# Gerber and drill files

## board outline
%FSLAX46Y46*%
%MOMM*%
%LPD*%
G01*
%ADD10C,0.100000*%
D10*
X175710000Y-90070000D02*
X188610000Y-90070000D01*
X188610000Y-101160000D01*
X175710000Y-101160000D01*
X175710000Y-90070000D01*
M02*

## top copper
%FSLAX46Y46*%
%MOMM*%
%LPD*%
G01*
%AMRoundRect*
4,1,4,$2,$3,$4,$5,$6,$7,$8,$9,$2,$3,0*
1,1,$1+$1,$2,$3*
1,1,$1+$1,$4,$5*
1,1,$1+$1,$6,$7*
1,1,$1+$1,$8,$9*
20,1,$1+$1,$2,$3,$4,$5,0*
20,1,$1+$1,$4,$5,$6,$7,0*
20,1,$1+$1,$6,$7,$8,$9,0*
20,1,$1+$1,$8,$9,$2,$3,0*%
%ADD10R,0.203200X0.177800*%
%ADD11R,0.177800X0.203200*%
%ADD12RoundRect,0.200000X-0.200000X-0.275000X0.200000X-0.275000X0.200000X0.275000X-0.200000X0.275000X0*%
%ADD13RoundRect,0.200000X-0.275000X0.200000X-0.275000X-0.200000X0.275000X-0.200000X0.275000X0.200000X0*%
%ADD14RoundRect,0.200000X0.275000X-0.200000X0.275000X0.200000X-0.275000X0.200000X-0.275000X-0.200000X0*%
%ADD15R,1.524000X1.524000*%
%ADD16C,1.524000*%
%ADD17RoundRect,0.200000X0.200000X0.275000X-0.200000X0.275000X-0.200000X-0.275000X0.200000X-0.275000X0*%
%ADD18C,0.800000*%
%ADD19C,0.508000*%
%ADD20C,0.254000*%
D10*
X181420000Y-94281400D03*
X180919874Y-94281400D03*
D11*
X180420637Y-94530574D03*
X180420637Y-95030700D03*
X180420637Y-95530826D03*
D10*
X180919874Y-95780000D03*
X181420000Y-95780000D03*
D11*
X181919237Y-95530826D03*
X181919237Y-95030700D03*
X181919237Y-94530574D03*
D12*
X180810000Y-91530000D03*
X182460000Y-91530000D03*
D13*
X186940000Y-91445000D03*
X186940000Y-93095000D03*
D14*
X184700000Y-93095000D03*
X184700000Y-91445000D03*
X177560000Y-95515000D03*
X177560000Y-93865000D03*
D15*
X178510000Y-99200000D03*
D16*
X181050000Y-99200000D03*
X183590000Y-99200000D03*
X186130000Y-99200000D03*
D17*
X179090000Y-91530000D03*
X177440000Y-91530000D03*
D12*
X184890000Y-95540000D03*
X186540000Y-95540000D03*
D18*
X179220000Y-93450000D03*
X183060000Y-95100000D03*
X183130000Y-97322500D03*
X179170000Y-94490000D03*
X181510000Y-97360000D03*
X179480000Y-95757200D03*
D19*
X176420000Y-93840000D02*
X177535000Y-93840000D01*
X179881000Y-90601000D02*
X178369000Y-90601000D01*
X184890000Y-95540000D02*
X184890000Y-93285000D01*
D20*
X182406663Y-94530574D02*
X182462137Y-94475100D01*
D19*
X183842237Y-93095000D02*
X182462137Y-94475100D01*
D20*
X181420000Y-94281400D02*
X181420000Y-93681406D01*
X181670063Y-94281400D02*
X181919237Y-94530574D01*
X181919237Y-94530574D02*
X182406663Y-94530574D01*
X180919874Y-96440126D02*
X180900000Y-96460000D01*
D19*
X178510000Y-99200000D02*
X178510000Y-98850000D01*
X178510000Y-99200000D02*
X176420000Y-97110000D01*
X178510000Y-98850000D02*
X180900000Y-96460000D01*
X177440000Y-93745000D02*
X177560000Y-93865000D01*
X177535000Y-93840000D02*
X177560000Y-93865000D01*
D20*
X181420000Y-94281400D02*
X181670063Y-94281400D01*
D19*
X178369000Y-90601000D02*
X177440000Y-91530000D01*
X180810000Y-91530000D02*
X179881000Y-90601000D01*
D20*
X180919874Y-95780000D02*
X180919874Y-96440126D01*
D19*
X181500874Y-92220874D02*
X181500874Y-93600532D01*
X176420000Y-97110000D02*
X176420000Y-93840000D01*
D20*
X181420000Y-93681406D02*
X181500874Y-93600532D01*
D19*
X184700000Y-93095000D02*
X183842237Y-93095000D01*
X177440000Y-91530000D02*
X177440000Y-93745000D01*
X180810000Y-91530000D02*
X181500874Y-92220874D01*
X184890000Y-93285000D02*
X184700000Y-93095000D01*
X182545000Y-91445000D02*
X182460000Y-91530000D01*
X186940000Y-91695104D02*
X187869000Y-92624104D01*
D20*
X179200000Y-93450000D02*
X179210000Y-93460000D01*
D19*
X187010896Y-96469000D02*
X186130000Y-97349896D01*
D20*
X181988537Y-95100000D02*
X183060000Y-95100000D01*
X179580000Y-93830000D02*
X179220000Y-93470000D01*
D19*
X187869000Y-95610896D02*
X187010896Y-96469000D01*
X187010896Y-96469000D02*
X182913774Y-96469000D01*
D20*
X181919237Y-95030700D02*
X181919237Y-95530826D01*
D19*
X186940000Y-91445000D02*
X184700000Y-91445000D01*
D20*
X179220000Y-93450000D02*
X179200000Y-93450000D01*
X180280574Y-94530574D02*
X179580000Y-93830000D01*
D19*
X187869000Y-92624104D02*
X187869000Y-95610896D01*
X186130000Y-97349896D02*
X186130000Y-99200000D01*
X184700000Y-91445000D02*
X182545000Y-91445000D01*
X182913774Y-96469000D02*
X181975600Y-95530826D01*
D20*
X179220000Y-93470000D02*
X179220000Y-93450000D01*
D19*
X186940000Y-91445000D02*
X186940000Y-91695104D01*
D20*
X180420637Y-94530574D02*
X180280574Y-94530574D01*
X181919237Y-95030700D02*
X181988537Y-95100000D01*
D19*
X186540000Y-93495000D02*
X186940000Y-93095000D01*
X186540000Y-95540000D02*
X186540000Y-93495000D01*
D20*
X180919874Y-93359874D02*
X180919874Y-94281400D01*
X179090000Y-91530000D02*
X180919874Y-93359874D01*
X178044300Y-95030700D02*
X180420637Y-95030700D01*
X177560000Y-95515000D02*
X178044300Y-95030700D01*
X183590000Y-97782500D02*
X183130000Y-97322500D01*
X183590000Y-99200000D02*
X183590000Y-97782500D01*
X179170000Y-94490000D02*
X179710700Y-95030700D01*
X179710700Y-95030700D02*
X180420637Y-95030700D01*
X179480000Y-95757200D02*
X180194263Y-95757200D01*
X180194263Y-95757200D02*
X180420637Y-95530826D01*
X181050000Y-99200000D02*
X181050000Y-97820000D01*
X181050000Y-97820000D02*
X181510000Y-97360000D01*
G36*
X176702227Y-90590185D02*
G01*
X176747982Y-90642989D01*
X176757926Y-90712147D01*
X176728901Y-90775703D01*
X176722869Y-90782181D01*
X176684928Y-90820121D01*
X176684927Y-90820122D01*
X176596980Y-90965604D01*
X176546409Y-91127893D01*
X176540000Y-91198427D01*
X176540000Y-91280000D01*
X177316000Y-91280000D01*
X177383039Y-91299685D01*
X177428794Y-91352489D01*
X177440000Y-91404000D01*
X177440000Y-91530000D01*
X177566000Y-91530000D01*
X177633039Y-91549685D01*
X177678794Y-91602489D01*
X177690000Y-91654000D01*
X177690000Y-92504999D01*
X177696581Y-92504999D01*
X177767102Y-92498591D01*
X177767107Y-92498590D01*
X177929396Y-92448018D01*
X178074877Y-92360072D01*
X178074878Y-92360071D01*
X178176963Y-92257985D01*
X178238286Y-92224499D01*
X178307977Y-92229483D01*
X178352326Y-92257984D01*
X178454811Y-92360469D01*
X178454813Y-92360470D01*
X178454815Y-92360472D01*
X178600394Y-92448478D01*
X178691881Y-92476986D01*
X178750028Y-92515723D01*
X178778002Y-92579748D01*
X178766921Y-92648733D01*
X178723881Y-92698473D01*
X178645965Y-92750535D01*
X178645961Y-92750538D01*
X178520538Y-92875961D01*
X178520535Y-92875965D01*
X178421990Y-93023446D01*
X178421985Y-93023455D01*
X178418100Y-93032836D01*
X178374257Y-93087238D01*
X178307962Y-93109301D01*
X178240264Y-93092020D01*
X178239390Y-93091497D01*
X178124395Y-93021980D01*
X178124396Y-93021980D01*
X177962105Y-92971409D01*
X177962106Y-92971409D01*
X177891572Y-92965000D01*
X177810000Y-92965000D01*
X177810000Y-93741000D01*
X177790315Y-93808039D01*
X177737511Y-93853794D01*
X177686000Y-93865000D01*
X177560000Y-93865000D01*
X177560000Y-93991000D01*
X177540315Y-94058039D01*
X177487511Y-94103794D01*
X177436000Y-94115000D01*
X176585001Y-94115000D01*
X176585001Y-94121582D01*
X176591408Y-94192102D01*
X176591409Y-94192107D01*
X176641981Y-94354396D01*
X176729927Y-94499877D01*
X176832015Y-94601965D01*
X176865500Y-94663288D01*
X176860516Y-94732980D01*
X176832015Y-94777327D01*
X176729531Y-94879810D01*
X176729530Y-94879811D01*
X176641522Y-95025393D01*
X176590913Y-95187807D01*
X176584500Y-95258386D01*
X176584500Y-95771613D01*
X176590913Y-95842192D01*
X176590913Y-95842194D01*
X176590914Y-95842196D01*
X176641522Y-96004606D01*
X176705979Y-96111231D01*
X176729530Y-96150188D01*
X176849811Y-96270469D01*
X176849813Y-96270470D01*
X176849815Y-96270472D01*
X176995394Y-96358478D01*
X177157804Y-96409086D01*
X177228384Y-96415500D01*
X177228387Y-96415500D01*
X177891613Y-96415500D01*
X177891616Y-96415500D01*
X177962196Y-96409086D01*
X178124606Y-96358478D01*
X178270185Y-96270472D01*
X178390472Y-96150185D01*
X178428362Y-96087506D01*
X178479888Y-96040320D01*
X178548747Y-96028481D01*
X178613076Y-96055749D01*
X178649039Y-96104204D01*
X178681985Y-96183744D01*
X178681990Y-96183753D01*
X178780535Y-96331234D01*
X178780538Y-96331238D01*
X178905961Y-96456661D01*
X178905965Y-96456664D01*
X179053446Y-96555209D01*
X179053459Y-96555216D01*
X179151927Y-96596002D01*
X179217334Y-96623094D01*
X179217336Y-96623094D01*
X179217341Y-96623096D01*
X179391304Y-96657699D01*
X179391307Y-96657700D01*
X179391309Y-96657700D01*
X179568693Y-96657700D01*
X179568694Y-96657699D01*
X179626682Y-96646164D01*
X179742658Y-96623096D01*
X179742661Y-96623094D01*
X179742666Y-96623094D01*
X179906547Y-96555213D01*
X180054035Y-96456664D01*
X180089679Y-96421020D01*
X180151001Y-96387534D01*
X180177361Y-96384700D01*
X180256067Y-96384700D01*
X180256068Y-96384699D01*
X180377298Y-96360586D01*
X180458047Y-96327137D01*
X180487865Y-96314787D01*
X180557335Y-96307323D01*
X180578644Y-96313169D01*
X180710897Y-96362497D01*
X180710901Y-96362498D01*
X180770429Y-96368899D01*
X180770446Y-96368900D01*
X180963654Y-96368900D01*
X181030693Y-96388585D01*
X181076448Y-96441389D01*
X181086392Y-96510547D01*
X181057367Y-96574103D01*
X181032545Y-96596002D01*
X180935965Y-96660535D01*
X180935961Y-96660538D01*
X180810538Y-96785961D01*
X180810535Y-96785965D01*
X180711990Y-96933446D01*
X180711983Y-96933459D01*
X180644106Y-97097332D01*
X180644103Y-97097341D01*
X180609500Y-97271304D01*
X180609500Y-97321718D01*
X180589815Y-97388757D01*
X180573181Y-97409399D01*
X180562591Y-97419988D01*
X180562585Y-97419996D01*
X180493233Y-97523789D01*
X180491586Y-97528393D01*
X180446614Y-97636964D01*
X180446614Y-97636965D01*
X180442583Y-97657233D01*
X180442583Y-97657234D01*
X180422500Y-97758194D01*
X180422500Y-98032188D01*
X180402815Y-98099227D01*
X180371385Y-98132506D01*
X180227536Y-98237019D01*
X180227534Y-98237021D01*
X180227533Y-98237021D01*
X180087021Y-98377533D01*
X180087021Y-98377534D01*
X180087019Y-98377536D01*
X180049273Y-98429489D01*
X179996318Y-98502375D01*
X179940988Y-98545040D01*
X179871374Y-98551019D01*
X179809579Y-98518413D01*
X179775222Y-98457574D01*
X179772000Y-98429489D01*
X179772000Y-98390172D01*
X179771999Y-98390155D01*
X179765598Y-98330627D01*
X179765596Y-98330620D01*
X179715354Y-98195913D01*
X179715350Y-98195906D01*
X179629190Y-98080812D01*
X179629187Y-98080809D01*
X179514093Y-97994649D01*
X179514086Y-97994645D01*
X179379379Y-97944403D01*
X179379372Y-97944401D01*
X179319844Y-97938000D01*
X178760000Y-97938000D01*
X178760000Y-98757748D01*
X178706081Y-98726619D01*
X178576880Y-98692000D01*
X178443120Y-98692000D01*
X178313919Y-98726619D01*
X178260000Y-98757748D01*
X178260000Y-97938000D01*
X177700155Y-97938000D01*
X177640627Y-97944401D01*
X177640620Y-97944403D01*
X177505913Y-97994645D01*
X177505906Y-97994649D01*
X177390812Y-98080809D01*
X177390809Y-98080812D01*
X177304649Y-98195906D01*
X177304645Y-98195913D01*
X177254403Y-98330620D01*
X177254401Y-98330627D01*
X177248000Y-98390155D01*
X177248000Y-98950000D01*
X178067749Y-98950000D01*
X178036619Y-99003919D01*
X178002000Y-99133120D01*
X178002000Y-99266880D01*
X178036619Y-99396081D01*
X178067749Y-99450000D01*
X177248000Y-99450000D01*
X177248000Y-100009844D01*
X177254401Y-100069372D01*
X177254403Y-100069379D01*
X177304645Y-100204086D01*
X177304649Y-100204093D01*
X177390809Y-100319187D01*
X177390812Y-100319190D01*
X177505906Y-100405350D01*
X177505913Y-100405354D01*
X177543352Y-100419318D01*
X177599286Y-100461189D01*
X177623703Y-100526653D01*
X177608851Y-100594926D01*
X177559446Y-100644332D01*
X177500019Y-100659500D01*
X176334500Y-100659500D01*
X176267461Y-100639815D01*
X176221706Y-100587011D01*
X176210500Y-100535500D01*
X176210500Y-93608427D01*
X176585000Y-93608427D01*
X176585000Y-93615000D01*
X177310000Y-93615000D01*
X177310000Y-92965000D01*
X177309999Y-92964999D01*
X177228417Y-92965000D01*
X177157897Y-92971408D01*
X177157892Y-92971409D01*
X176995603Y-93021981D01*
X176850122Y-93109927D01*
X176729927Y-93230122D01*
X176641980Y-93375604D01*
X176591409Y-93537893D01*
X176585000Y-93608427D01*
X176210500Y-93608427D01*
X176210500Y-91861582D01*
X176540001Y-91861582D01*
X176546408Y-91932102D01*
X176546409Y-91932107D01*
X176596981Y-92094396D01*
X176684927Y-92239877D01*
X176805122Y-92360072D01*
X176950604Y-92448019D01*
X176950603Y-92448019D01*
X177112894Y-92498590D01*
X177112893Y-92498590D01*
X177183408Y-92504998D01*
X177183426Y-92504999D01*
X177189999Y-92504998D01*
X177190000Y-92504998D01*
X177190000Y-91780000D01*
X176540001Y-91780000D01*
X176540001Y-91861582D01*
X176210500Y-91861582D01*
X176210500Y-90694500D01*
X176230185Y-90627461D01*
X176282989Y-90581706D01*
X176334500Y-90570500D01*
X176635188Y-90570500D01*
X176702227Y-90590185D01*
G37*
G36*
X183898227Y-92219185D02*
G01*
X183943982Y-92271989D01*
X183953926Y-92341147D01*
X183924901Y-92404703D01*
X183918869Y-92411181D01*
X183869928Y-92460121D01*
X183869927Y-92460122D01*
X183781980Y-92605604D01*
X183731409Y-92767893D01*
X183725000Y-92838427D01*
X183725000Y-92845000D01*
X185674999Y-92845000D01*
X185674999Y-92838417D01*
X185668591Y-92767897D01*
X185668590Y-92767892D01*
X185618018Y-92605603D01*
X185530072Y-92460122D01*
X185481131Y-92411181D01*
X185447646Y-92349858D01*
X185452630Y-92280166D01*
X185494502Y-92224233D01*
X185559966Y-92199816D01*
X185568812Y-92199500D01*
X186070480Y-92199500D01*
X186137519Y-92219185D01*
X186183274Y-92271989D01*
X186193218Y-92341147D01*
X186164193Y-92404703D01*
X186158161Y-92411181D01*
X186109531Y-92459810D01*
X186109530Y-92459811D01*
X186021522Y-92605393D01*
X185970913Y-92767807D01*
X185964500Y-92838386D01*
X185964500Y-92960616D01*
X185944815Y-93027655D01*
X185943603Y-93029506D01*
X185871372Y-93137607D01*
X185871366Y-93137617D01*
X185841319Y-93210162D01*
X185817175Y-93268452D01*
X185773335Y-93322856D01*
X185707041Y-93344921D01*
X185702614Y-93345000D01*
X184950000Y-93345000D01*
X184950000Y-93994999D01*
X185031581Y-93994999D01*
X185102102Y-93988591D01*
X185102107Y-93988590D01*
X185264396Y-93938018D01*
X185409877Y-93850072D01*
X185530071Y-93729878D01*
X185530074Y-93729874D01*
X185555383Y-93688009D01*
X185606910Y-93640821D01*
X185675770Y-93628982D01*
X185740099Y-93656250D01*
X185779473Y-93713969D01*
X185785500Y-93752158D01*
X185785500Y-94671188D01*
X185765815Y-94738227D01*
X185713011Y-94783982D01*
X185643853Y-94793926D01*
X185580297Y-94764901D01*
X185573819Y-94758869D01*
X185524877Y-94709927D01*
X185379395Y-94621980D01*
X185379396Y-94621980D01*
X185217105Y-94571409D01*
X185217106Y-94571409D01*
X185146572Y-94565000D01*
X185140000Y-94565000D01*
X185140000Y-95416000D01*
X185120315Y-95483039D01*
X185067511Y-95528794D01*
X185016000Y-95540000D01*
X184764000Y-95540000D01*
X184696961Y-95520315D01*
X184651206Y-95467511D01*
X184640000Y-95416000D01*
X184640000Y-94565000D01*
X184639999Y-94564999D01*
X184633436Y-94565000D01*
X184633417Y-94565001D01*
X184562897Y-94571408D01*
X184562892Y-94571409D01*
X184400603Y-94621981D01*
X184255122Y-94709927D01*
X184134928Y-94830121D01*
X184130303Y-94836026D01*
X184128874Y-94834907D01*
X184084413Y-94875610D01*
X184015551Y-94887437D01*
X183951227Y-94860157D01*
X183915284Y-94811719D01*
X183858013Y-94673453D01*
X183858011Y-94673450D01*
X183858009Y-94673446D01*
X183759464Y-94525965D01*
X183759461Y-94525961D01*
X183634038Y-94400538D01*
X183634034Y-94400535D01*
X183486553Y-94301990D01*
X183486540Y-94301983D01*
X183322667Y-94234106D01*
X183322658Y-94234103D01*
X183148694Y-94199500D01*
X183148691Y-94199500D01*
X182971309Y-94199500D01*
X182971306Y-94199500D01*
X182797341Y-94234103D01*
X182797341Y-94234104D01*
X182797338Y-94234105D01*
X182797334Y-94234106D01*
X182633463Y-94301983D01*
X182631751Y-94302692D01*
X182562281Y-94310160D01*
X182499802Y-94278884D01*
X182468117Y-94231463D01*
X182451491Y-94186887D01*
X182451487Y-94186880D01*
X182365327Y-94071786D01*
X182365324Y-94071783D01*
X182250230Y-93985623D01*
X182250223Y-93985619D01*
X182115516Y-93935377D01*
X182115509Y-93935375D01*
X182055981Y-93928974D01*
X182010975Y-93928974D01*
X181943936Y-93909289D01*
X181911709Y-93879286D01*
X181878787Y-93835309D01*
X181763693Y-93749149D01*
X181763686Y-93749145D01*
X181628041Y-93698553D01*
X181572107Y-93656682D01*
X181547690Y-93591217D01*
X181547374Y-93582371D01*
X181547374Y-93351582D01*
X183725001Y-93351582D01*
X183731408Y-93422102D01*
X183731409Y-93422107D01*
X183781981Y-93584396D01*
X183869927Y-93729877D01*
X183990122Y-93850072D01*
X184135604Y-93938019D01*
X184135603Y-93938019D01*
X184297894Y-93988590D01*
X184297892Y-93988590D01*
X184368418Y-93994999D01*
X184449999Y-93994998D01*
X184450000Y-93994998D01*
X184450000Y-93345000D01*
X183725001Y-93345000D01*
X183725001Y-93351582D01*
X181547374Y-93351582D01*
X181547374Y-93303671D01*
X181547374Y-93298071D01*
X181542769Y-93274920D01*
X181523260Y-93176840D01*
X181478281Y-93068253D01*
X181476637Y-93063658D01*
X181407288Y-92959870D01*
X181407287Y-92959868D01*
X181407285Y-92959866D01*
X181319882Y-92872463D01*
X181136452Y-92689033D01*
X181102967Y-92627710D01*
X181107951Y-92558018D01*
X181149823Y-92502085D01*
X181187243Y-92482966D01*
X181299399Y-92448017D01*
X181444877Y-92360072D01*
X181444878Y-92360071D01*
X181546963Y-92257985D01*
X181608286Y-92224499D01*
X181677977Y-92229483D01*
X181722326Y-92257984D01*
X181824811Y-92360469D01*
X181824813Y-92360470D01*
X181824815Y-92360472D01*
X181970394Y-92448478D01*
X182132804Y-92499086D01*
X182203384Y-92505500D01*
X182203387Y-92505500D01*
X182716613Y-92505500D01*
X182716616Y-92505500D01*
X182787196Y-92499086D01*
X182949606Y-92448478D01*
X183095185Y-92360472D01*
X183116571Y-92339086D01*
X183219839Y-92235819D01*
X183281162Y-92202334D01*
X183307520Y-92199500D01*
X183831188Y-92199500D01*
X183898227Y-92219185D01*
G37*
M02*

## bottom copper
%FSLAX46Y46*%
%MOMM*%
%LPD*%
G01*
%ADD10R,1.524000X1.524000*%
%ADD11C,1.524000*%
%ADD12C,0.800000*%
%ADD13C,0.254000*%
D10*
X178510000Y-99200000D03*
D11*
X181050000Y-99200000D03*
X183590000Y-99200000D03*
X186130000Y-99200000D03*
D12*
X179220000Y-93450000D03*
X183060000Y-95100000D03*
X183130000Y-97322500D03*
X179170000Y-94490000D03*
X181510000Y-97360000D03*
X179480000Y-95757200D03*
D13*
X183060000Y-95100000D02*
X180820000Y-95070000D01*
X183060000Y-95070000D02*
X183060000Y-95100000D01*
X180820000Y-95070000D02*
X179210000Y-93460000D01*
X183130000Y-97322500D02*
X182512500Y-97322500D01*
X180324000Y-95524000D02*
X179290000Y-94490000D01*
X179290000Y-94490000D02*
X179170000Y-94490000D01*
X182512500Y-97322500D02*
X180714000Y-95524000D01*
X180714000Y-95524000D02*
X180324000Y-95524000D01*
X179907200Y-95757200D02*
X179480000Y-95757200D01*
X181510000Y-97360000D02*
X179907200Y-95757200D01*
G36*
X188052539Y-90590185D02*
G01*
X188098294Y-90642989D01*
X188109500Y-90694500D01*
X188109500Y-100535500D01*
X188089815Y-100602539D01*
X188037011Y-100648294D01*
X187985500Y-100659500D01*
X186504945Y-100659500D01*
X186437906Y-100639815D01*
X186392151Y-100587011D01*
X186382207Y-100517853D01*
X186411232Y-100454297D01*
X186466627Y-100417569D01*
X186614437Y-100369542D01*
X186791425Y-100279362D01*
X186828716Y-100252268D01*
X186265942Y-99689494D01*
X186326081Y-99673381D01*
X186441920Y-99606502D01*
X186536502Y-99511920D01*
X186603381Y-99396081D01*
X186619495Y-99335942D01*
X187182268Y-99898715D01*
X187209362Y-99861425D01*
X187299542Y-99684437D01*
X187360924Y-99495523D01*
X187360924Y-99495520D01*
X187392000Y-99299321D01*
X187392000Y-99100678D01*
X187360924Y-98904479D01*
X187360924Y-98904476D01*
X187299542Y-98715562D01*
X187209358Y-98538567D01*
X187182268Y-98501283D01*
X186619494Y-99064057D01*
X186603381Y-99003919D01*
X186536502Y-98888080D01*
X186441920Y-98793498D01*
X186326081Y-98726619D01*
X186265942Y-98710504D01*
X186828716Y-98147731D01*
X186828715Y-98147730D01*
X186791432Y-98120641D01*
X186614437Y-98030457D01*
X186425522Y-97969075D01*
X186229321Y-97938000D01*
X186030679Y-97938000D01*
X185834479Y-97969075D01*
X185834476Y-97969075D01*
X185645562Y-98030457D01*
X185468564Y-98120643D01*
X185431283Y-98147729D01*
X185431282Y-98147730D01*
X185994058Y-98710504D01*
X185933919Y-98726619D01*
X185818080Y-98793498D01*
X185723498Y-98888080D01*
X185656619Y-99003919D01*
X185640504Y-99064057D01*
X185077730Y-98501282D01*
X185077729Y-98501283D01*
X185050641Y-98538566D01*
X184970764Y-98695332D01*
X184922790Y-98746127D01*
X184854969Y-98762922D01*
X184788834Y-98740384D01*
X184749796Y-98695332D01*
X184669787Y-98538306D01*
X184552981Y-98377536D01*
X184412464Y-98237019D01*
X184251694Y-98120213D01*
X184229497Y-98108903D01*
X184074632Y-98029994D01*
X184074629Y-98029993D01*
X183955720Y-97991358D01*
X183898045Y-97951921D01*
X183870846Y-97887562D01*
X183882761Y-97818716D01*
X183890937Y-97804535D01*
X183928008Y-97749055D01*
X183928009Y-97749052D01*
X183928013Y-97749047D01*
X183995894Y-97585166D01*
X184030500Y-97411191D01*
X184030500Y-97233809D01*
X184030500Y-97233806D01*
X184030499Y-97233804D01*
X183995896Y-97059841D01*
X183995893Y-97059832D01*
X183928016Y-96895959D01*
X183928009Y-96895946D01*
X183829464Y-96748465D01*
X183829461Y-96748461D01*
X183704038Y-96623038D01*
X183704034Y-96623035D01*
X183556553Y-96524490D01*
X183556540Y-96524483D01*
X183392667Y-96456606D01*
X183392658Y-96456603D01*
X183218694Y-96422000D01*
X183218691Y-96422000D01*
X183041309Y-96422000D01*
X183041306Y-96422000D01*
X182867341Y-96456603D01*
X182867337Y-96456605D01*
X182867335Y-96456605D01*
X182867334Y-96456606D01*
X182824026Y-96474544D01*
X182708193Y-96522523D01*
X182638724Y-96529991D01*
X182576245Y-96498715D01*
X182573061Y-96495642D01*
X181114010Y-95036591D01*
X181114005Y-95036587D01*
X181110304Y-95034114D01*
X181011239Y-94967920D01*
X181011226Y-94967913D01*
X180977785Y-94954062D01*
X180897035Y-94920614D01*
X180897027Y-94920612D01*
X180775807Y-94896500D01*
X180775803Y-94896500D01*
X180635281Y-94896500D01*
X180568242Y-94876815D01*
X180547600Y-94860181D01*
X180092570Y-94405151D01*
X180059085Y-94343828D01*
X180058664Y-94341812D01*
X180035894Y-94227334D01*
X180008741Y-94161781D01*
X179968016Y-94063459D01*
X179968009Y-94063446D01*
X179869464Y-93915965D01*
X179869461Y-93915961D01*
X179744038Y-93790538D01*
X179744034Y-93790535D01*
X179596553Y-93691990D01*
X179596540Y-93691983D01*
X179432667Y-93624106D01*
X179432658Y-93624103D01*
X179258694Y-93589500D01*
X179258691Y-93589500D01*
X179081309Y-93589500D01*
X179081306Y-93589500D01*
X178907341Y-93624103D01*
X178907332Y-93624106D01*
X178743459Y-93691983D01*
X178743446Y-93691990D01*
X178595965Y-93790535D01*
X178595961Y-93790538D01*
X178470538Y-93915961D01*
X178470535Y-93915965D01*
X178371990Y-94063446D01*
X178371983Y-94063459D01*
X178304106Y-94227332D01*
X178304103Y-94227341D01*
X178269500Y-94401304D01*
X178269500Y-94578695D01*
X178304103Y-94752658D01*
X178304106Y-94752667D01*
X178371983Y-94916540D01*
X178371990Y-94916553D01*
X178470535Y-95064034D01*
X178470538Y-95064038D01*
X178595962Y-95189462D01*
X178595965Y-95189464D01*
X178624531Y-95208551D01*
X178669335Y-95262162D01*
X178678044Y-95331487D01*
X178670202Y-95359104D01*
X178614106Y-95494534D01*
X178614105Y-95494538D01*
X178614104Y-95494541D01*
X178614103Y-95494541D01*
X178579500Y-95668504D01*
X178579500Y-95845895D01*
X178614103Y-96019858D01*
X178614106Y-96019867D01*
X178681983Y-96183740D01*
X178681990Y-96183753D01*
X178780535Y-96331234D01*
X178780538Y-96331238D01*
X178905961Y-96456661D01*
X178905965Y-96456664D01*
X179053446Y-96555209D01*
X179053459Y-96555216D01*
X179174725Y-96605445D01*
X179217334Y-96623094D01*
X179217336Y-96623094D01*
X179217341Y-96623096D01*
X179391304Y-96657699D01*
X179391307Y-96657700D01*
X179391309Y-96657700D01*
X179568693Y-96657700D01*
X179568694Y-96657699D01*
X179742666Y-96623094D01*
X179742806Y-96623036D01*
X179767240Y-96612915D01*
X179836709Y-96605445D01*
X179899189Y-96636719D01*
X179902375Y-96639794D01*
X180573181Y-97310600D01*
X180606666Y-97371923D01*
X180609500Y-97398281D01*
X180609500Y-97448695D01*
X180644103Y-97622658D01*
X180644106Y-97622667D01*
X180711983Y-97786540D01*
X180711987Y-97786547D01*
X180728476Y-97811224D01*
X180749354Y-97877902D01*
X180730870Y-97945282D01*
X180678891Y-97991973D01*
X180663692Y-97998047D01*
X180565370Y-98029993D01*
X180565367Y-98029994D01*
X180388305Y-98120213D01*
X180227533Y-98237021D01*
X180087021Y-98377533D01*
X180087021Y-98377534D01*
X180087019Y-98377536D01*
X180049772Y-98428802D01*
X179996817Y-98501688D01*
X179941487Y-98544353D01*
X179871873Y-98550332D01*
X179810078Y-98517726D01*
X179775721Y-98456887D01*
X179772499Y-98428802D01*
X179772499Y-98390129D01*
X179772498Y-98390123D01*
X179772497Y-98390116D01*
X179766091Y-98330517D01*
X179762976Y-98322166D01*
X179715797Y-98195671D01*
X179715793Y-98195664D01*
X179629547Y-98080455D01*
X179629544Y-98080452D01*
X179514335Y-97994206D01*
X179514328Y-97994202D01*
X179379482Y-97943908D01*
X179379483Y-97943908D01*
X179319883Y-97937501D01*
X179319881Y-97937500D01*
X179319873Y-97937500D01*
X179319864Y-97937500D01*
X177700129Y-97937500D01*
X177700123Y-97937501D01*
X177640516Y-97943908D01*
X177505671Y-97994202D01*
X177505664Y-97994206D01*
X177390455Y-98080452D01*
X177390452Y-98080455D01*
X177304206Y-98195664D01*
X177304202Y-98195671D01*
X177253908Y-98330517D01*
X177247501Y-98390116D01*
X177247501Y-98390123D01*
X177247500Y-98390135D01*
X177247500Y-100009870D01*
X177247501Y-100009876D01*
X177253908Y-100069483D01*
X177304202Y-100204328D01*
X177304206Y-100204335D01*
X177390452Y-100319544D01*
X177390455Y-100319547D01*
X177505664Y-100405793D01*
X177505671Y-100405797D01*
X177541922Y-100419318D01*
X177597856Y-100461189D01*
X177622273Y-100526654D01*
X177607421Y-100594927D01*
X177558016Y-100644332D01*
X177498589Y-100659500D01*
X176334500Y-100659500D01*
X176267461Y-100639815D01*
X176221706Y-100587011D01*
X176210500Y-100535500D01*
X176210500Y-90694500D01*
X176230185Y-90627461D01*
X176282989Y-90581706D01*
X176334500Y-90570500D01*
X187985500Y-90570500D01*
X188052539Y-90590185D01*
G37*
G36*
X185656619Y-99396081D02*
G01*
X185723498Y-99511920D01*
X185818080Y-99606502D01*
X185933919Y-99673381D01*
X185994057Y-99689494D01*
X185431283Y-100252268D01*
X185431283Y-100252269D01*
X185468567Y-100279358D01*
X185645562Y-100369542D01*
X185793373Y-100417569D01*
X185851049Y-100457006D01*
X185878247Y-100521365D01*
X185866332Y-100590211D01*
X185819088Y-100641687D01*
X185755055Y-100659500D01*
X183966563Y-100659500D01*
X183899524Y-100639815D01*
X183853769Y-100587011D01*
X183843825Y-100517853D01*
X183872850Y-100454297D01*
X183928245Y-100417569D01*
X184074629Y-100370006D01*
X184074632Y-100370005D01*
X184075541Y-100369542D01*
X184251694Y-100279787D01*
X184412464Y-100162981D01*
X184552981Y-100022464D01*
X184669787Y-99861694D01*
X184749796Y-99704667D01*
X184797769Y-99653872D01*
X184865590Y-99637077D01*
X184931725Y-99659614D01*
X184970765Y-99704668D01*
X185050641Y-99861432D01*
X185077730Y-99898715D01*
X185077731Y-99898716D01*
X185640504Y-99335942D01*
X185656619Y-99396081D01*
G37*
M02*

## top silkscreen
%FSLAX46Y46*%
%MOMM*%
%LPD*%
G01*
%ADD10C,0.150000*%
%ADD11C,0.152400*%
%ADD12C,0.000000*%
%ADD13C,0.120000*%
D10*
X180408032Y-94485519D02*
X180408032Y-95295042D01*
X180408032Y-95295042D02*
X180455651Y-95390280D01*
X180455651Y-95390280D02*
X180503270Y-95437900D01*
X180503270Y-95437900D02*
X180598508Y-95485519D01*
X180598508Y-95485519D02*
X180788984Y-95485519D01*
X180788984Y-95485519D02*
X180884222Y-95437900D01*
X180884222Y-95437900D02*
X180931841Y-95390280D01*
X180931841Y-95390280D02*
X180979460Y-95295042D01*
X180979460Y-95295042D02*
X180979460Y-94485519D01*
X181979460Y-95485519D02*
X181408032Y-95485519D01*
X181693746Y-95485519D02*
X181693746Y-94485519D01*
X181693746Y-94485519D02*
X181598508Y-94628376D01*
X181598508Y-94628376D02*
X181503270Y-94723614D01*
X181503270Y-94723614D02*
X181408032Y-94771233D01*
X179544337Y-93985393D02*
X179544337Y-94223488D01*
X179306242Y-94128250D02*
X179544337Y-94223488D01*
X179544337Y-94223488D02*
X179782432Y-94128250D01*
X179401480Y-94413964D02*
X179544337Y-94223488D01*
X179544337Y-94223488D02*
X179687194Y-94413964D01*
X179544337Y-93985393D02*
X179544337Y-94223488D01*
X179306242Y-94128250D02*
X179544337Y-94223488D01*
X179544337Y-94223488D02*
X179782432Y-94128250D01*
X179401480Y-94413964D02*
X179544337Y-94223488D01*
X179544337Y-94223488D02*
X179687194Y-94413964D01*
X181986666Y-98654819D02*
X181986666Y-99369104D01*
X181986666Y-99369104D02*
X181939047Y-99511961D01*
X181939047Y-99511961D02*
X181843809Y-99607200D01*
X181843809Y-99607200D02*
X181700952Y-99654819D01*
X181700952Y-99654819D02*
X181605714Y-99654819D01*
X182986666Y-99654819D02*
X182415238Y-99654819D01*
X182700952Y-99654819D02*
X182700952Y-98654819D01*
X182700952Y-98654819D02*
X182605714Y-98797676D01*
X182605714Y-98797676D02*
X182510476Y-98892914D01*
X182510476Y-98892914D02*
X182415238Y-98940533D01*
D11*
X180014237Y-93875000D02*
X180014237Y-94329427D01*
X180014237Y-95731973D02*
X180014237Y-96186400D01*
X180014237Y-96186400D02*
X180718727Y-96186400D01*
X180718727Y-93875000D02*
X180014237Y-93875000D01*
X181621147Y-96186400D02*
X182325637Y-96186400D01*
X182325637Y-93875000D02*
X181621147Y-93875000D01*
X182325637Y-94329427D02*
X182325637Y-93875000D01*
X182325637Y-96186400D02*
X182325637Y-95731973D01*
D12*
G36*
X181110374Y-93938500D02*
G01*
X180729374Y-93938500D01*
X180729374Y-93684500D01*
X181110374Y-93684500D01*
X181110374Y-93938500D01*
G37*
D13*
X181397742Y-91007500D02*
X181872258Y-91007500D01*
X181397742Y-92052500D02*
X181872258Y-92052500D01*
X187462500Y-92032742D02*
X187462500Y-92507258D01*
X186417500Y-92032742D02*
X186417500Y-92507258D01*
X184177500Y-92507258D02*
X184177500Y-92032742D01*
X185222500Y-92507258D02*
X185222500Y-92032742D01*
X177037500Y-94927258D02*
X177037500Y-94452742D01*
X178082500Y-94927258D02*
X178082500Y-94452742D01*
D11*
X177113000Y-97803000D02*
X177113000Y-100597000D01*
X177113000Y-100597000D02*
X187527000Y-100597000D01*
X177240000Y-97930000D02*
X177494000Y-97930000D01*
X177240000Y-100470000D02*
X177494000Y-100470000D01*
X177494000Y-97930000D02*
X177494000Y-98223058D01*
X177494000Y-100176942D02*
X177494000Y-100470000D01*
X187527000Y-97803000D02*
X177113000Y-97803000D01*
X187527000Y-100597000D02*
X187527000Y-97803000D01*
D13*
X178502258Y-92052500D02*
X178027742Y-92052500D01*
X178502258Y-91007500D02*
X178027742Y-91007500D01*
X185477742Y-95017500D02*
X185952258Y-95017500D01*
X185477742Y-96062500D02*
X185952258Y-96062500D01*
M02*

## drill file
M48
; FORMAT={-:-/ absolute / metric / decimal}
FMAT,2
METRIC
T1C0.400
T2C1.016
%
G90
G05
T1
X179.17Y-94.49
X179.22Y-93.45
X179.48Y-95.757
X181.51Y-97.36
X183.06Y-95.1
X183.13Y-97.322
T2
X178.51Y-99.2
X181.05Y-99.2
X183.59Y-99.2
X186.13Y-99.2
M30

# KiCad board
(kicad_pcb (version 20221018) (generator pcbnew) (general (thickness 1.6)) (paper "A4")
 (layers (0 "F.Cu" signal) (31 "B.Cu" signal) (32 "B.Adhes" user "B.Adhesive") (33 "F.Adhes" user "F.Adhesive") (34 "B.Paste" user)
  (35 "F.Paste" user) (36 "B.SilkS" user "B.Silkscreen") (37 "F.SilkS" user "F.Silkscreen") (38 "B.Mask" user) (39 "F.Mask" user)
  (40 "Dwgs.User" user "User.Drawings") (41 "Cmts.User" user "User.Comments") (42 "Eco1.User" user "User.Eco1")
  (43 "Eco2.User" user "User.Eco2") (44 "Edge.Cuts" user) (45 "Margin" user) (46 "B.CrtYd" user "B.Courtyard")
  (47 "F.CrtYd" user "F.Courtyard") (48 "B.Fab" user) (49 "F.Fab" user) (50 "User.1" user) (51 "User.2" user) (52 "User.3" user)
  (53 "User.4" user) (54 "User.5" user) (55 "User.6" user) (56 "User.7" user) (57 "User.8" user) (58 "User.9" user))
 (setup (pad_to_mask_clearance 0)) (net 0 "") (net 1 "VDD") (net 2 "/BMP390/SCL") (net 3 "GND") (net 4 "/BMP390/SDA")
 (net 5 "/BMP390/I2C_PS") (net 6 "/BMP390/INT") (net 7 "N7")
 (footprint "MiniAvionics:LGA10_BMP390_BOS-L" (layer "F.Cu") (at 181.169937 95.0307)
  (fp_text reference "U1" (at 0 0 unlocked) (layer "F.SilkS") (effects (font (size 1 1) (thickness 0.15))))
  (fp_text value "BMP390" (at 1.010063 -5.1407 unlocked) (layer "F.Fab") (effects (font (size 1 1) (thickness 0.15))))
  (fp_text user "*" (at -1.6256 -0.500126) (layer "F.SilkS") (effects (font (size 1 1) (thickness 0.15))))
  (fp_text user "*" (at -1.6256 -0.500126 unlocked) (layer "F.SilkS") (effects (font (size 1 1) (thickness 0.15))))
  (fp_line (start -1.1557 -1.1557) (end -1.1557 -0.701273) (stroke (width 0.1524) (type solid)) (layer "F.SilkS"))
  (fp_line (start -1.1557 0.701273) (end -1.1557 1.1557) (stroke (width 0.1524) (type solid)) (layer "F.SilkS"))
  (fp_line (start -1.1557 1.1557) (end -0.45121 1.1557) (stroke (width 0.1524) (type solid)) (layer "F.SilkS"))
  (fp_line (start -0.45121 -1.1557) (end -1.1557 -1.1557) (stroke (width 0.1524) (type solid)) (layer "F.SilkS"))
  (fp_line (start 0.45121 1.1557) (end 1.1557 1.1557) (stroke (width 0.1524) (type solid)) (layer "F.SilkS"))
  (fp_line (start 1.1557 -1.1557) (end 0.45121 -1.1557) (stroke (width 0.1524) (type solid)) (layer "F.SilkS"))
  (fp_line (start 1.1557 -0.701273) (end 1.1557 -1.1557) (stroke (width 0.1524) (type solid)) (layer "F.SilkS"))
  (fp_line (start 1.1557 1.1557) (end 1.1557 0.701273) (stroke (width 0.1524) (type solid)) (layer "F.SilkS"))
  (fp_poly
   (pts (xy -0.440563 -1.0922) (xy -0.440563 -1.3462) (xy -0.059563 -1.3462) (xy -0.059563 -1.0922)) (stroke (width 0) (type solid))
   (fill solid) (layer "F.SilkS"))
  (pad "1" smd rect (at 0.250063 -0.7493) (size 0.2032 0.1778) (layers "F.Cu" "F.Paste" "F.Mask") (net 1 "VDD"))
  (pad "2" smd rect (at -0.250063 -0.7493) (size 0.2032 0.1778) (layers "F.Cu" "F.Paste" "F.Mask") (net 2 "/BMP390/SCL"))
  (pad "3" smd rect (at -0.7493 -0.500126 90) (size 0.2032 0.1778) (layers "F.Cu" "F.Paste" "F.Mask") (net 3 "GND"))
  (pad "4" smd rect (at -0.7493 0 90) (size 0.2032 0.1778) (layers "F.Cu" "F.Paste" "F.Mask") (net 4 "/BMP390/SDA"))
  (pad "5" smd rect (at -0.7493 0.500126 90) (size 0.2032 0.1778) (layers "F.Cu" "F.Paste" "F.Mask") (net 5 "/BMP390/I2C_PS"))
  (pad "6" smd rect (at -0.250063 0.7493) (size 0.2032 0.1778) (layers "F.Cu" "F.Paste" "F.Mask") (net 1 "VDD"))
  (pad "7" smd rect (at 0.250063 0.7493) (size 0.2032 0.1778) (layers "F.Cu" "F.Paste" "F.Mask") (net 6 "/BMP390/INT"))
  (pad "8" smd rect (at 0.7493 0.500126 90) (size 0.2032 0.1778) (layers "F.Cu" "F.Paste" "F.Mask") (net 3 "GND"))
  (pad "9" smd rect (at 0.7493 0 90) (size 0.2032 0.1778) (layers "F.Cu" "F.Paste" "F.Mask") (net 3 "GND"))
  (pad "10" smd rect (at 0.7493 -0.500126 90) (size 0.2032 0.1778) (layers "F.Cu" "F.Paste" "F.Mask") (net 1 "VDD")))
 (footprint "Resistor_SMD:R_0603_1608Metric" (layer "F.Cu") (at 181.635 91.53)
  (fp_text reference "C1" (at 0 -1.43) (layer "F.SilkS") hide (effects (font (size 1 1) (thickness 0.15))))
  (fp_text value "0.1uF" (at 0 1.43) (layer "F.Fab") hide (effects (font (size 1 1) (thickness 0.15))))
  (fp_line (start -0.237258 -0.5225) (end 0.237258 -0.5225) (stroke (width 0.12) (type solid)) (layer "F.SilkS"))
  (fp_line (start -0.237258 0.5225) (end 0.237258 0.5225) (stroke (width 0.12) (type solid)) (layer "F.SilkS"))
  (pad "1" smd roundrect (at -0.825 0) (size 0.8 0.95) (layers "F.Cu" "F.Paste" "F.Mask") (roundrect_rratio 0.25) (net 1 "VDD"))
  (pad "2" smd roundrect (at 0.825 0) (size 0.8 0.95) (layers "F.Cu" "F.Paste" "F.Mask") (roundrect_rratio 0.25) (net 3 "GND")))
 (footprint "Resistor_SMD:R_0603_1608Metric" (layer "F.Cu") (at 186.94 92.27 -90)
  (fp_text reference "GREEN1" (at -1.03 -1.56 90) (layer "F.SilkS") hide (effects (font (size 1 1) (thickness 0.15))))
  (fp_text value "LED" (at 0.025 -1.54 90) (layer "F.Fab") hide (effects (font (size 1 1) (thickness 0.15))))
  (fp_line (start -0.237258 -0.5225) (end 0.237258 -0.5225) (stroke (width 0.12) (type solid)) (layer "F.SilkS"))
  (fp_line (start -0.237258 0.5225) (end 0.237258 0.5225) (stroke (width 0.12) (type solid)) (layer "F.SilkS"))
  (pad "1" smd roundrect (at -0.825 0 270) (size 0.8 0.95) (layers "F.Cu" "F.Paste" "F.Mask") (roundrect_rratio 0.25) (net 3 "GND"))
  (pad "2" smd roundrect (at 0.825 0 270) (size 0.8 0.95) (layers "F.Cu" "F.Paste" "F.Mask") (roundrect_rratio 0.25) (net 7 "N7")))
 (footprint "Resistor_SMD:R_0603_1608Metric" (layer "F.Cu") (at 184.7 92.27 90)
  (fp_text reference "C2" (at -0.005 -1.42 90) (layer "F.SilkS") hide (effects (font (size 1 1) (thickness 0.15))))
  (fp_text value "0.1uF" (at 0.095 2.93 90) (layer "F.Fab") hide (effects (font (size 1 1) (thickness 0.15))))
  (fp_line (start -0.237258 -0.5225) (end 0.237258 -0.5225) (stroke (width 0.12) (type solid)) (layer "F.SilkS"))
  (fp_line (start -0.237258 0.5225) (end 0.237258 0.5225) (stroke (width 0.12) (type solid)) (layer "F.SilkS"))
  (pad "1" smd roundrect (at -0.825 0 90) (size 0.8 0.95) (layers "F.Cu" "F.Paste" "F.Mask") (roundrect_rratio 0.25) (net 1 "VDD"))
  (pad "2" smd roundrect (at 0.825 0 90) (size 0.8 0.95) (layers "F.Cu" "F.Paste" "F.Mask") (roundrect_rratio 0.25) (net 3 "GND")))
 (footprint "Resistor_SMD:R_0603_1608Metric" (layer "F.Cu") (at 177.56 94.69 90)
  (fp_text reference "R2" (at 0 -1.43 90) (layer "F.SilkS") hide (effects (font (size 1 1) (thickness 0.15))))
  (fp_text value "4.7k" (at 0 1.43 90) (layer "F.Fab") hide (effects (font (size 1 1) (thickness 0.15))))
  (fp_line (start -0.237258 -0.5225) (end 0.237258 -0.5225) (stroke (width 0.12) (type solid)) (layer "F.SilkS"))
  (fp_line (start -0.237258 0.5225) (end 0.237258 0.5225) (stroke (width 0.12) (type solid)) (layer "F.SilkS"))
  (pad "1" smd roundrect (at -0.825 0 90) (size 0.8 0.95) (layers "F.Cu" "F.Paste" "F.Mask") (roundrect_rratio 0.25) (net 4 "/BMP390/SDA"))
  (pad "2" smd roundrect (at 0.825 0 90) (size 0.8 0.95) (layers "F.Cu" "F.Paste" "F.Mask") (roundrect_rratio 0.25) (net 1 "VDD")))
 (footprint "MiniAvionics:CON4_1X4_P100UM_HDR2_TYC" (layer "F.Cu") (at 178.51 99.2)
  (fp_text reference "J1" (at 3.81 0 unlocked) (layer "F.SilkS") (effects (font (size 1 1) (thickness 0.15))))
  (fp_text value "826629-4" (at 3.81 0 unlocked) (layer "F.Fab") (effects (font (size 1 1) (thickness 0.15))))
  (fp_line (start -1.397 -1.397) (end -1.397 1.397) (stroke (width 0.1524) (type solid)) (layer "F.SilkS"))
  (fp_line (start -1.397 1.397) (end 9.017 1.397) (stroke (width 0.1524) (type solid)) (layer "F.SilkS"))
  (fp_line (start -1.27 -1.27) (end -1.016 -1.27) (stroke (width 0.1524) (type solid)) (layer "F.SilkS"))
  (fp_line (start -1.27 1.27) (end -1.016 1.27) (stroke (width 0.1524) (type solid)) (layer "F.SilkS"))
  (fp_line (start -1.016 -1.27) (end -1.016 -0.976942) (stroke (width 0.1524) (type solid)) (layer "F.SilkS"))
  (fp_line (start -1.016 0.976942) (end -1.016 1.27) (stroke (width 0.1524) (type solid)) (layer "F.SilkS"))
  (fp_line (start 9.017 -1.397) (end -1.397 -1.397) (stroke (width 0.1524) (type solid)) (layer "F.SilkS"))
  (fp_line (start 9.017 1.397) (end 9.017 -1.397) (stroke (width 0.1524) (type solid)) (layer "F.SilkS"))
  (pad "1" thru_hole rect (at 0 0) (size 1.524 1.524) (drill 1.016) (layers "*.Cu" "*.Mask") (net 1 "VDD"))
  (pad "2" thru_hole circle (at 2.54 0) (size 1.524 1.524) (drill 1.016) (layers "*.Cu" "*.Mask") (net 5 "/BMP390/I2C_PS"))
  (pad "3" thru_hole circle (at 5.08 0) (size 1.524 1.524) (drill 1.016) (layers "*.Cu" "*.Mask") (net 4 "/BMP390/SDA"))
  (pad "4" thru_hole circle (at 7.62 0) (size 1.524 1.524) (drill 1.016) (layers "*.Cu" "*.Mask") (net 3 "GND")))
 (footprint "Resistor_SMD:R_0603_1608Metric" (layer "F.Cu") (at 178.265 91.53 180)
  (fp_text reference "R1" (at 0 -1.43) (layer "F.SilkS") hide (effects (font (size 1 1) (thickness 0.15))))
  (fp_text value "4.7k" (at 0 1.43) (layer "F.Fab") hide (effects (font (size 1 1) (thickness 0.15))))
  (fp_line (start -0.237258 -0.5225) (end 0.237258 -0.5225) (stroke (width 0.12) (type solid)) (layer "F.SilkS"))
  (fp_line (start -0.237258 0.5225) (end 0.237258 0.5225) (stroke (width 0.12) (type solid)) (layer "F.SilkS"))
  (pad "1" smd roundrect (at -0.825 0 180) (size 0.8 0.95) (layers "F.Cu" "F.Paste" "F.Mask") (roundrect_rratio 0.25) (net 2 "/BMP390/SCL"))
  (pad "2" smd roundrect (at 0.825 0 180) (size 0.8 0.95) (layers "F.Cu" "F.Paste" "F.Mask") (roundrect_rratio 0.25) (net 1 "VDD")))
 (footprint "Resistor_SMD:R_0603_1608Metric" (layer "F.Cu") (at 185.715 95.54)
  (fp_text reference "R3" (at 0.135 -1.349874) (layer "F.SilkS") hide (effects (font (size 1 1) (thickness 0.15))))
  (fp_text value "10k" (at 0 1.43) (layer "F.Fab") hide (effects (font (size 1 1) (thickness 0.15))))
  (fp_line (start -0.237258 -0.5225) (end 0.237258 -0.5225) (stroke (width 0.12) (type solid)) (layer "F.SilkS"))
  (fp_line (start -0.237258 0.5225) (end 0.237258 0.5225) (stroke (width 0.12) (type solid)) (layer "F.SilkS"))
  (pad "1" smd roundrect (at -0.825 0) (size 0.8 0.95) (layers "F.Cu" "F.Paste" "F.Mask") (roundrect_rratio 0.25) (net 1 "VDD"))
  (pad "2" smd roundrect (at 0.825 0) (size 0.8 0.95) (layers "F.Cu" "F.Paste" "F.Mask") (roundrect_rratio 0.25) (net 7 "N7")))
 (gr_rect (start 175.71 90.07) (end 188.61 101.16) (stroke (width 0.1) (type default)) (fill none) (layer "Edge.Cuts"))
 (segment (start 176.42 93.84) (end 177.535 93.84) (width 0.508) (layer "F.Cu") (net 1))
 (segment (start 179.881 90.601) (end 178.369 90.601) (width 0.508) (layer "F.Cu") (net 1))
 (segment (start 184.89 95.54) (end 184.89 93.285) (width 0.508) (layer "F.Cu") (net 1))
 (segment (start 182.406663 94.530574) (end 182.462137 94.4751) (width 0.254) (layer "F.Cu") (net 1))
 (segment (start 183.842237 93.095) (end 182.462137 94.4751) (width 0.508) (layer "F.Cu") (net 1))
 (segment (start 181.42 94.2814) (end 181.42 93.681406) (width 0.254) (layer "F.Cu") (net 1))
 (segment (start 181.670063 94.2814) (end 181.919237 94.530574) (width 0.254) (layer "F.Cu") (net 1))
 (segment (start 181.919237 94.530574) (end 182.406663 94.530574) (width 0.254) (layer "F.Cu") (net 1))
 (segment (start 180.919874 96.440126) (end 180.9 96.46) (width 0.254) (layer "F.Cu") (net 1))
 (segment (start 178.51 99.2) (end 178.51 98.85) (width 0.508) (layer "F.Cu") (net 1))
 (segment (start 178.51 99.2) (end 176.42 97.11) (width 0.508) (layer "F.Cu") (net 1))
 (segment (start 178.51 98.85) (end 180.9 96.46) (width 0.508) (layer "F.Cu") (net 1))
 (segment (start 177.44 93.745) (end 177.56 93.865) (width 0.508) (layer "F.Cu") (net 1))
 (segment (start 177.535 93.84) (end 177.56 93.865) (width 0.508) (layer "F.Cu") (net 1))
 (segment (start 181.42 94.2814) (end 181.670063 94.2814) (width 0.254) (layer "F.Cu") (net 1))
 (segment (start 178.369 90.601) (end 177.44 91.53) (width 0.508) (layer "F.Cu") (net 1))
 (segment (start 180.81 91.53) (end 179.881 90.601) (width 0.508) (layer "F.Cu") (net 1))
 (segment (start 180.919874 95.78) (end 180.919874 96.440126) (width 0.254) (layer "F.Cu") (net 1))
 (segment (start 181.500874 92.220874) (end 181.500874 93.600532) (width 0.508) (layer "F.Cu") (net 1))
 (segment (start 176.42 97.11) (end 176.42 93.84) (width 0.508) (layer "F.Cu") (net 1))
 (segment (start 181.42 93.681406) (end 181.500874 93.600532) (width 0.254) (layer "F.Cu") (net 1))
 (segment (start 184.7 93.095) (end 183.842237 93.095) (width 0.508) (layer "F.Cu") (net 1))
 (segment (start 177.44 91.53) (end 177.44 93.745) (width 0.508) (layer "F.Cu") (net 1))
 (segment (start 180.81 91.53) (end 181.500874 92.220874) (width 0.508) (layer "F.Cu") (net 1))
 (segment (start 184.89 93.285) (end 184.7 93.095) (width 0.508) (layer "F.Cu") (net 1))
 (segment (start 182.545 91.445) (end 182.46 91.53) (width 0.508) (layer "F.Cu") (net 3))
 (segment (start 186.94 91.695104) (end 187.869 92.624104) (width 0.508) (layer "F.Cu") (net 3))
 (segment (start 179.2 93.45) (end 179.21 93.46) (width 0.254) (layer "F.Cu") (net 3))
 (segment (start 187.010896 96.469) (end 186.13 97.349896) (width 0.508) (layer "F.Cu") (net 3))
 (segment (start 181.988537 95.1) (end 183.06 95.1) (width 0.254) (layer "F.Cu") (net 3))
 (segment (start 179.58 93.83) (end 179.22 93.47) (width 0.254) (layer "F.Cu") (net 3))
 (segment (start 187.869 95.610896) (end 187.010896 96.469) (width 0.508) (layer "F.Cu") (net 3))
 (segment (start 187.010896 96.469) (end 182.913774 96.469) (width 0.508) (layer "F.Cu") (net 3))
 (segment (start 181.919237 95.0307) (end 181.919237 95.530826) (width 0.254) (layer "F.Cu") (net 3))
 (segment (start 186.94 91.445) (end 184.7 91.445) (width 0.508) (layer "F.Cu") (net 3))
 (segment (start 179.22 93.45) (end 179.2 93.45) (width 0.254) (layer "F.Cu") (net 3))
 (segment (start 180.280574 94.530574) (end 179.58 93.83) (width 0.254) (layer "F.Cu") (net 3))
 (segment (start 187.869 92.624104) (end 187.869 95.610896) (width 0.508) (layer "F.Cu") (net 3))
 (segment (start 186.13 97.349896) (end 186.13 99.2) (width 0.508) (layer "F.Cu") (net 3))
 (segment (start 184.7 91.445) (end 182.545 91.445) (width 0.508) (layer "F.Cu") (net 3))
 (segment (start 182.913774 96.469) (end 181.9756 95.530826) (width 0.508) (layer "F.Cu") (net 3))
 (segment (start 179.22 93.47) (end 179.22 93.45) (width 0.254) (layer "F.Cu") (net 3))
 (segment (start 186.94 91.445) (end 186.94 91.695104) (width 0.508) (layer "F.Cu") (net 3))
 (segment (start 180.420637 94.530574) (end 180.280574 94.530574) (width 0.254) (layer "F.Cu") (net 3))
 (segment (start 181.919237 95.0307) (end 181.988537 95.1) (width 0.254) (layer "F.Cu") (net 3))
 (via (at 179.22 93.45) (size 0.8) (drill 0.4) (layers "F.Cu" "B.Cu") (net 3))
 (via (at 183.06 95.1) (size 0.8) (drill 0.4) (layers "F.Cu" "B.Cu") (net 3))
 (segment (start 183.06 95.1) (end 180.82 95.07) (width 0.254) (layer "B.Cu") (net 3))
 (segment (start 183.06 95.07) (end 183.06 95.1) (width 0.254) (layer "B.Cu") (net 3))
 (segment (start 180.82 95.07) (end 179.21 93.46) (width 0.254) (layer "B.Cu") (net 3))
 (segment (start 186.54 93.495) (end 186.94 93.095) (width 0.508) (layer "F.Cu") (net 7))
 (segment (start 186.54 95.54) (end 186.54 93.495) (width 0.508) (layer "F.Cu") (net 7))
 (segment (start 180.919874 93.359874) (end 180.919874 94.2814) (width 0.254) (layer "F.Cu") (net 2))
 (segment (start 179.09 91.53) (end 180.919874 93.359874) (width 0.254) (layer "F.Cu") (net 2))
 (segment (start 178.0443 95.0307) (end 180.420637 95.0307) (width 0.254) (layer "F.Cu") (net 4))
 (segment (start 177.56 95.515) (end 178.0443 95.0307) (width 0.254) (layer "F.Cu") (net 4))
 (segment (start 183.59 97.7825) (end 183.13 97.3225) (width 0.254) (layer "F.Cu") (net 4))
 (segment (start 183.59 99.2) (end 183.59 97.7825) (width 0.254) (layer "F.Cu") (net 4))
 (segment (start 179.17 94.49) (end 179.7107 95.0307) (width 0.254) (layer "F.Cu") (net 4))
 (segment (start 179.7107 95.0307) (end 180.420637 95.0307) (width 0.254) (layer "F.Cu") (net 4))
 (via (at 183.13 97.3225) (size 0.8) (drill 0.4) (layers "F.Cu" "B.Cu") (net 4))
 (via (at 179.17 94.49) (size 0.8) (drill 0.4) (layers "F.Cu" "B.Cu") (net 4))
 (segment (start 183.13 97.3225) (end 182.5125 97.3225) (width 0.254) (layer "B.Cu") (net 4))
 (segment (start 180.324 95.524) (end 179.29 94.49) (width 0.254) (layer "B.Cu") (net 4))
 (segment (start 179.29 94.49) (end 179.17 94.49) (width 0.254) (layer "B.Cu") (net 4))
 (segment (start 182.5125 97.3225) (end 180.714 95.524) (width 0.254) (layer "B.Cu") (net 4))
 (segment (start 180.714 95.524) (end 180.324 95.524) (width 0.254) (layer "B.Cu") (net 4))
 (segment (start 179.48 95.7572) (end 180.194263 95.7572) (width 0.254) (layer "F.Cu") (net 5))
 (segment (start 180.194263 95.7572) (end 180.420637 95.530826) (width 0.254) (layer "F.Cu") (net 5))
 (segment (start 181.05 99.2) (end 181.05 97.82) (width 0.254) (layer "F.Cu") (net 5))
 (segment (start 181.05 97.82) (end 181.51 97.36) (width 0.254) (layer "F.Cu") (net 5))
 (via (at 181.51 97.36) (size 0.8) (drill 0.4) (layers "F.Cu" "B.Cu") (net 5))
 (via (at 179.48 95.7572) (size 0.8) (drill 0.4) (layers "F.Cu" "B.Cu") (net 5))
 (segment (start 179.9072 95.7572) (end 179.48 95.7572) (width 0.254) (layer "B.Cu") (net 5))
 (segment (start 181.51 97.36) (end 179.9072 95.7572) (width 0.254) (layer "B.Cu") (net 5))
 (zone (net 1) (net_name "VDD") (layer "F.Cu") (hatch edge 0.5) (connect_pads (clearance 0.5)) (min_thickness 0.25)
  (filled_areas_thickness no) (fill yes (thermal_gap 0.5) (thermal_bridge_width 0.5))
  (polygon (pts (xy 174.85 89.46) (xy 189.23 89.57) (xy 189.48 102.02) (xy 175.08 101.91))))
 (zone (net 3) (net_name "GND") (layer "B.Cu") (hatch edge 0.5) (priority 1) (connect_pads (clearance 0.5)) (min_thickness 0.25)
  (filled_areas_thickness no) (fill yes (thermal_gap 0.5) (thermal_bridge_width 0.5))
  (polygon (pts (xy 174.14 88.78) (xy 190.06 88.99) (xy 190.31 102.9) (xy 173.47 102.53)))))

